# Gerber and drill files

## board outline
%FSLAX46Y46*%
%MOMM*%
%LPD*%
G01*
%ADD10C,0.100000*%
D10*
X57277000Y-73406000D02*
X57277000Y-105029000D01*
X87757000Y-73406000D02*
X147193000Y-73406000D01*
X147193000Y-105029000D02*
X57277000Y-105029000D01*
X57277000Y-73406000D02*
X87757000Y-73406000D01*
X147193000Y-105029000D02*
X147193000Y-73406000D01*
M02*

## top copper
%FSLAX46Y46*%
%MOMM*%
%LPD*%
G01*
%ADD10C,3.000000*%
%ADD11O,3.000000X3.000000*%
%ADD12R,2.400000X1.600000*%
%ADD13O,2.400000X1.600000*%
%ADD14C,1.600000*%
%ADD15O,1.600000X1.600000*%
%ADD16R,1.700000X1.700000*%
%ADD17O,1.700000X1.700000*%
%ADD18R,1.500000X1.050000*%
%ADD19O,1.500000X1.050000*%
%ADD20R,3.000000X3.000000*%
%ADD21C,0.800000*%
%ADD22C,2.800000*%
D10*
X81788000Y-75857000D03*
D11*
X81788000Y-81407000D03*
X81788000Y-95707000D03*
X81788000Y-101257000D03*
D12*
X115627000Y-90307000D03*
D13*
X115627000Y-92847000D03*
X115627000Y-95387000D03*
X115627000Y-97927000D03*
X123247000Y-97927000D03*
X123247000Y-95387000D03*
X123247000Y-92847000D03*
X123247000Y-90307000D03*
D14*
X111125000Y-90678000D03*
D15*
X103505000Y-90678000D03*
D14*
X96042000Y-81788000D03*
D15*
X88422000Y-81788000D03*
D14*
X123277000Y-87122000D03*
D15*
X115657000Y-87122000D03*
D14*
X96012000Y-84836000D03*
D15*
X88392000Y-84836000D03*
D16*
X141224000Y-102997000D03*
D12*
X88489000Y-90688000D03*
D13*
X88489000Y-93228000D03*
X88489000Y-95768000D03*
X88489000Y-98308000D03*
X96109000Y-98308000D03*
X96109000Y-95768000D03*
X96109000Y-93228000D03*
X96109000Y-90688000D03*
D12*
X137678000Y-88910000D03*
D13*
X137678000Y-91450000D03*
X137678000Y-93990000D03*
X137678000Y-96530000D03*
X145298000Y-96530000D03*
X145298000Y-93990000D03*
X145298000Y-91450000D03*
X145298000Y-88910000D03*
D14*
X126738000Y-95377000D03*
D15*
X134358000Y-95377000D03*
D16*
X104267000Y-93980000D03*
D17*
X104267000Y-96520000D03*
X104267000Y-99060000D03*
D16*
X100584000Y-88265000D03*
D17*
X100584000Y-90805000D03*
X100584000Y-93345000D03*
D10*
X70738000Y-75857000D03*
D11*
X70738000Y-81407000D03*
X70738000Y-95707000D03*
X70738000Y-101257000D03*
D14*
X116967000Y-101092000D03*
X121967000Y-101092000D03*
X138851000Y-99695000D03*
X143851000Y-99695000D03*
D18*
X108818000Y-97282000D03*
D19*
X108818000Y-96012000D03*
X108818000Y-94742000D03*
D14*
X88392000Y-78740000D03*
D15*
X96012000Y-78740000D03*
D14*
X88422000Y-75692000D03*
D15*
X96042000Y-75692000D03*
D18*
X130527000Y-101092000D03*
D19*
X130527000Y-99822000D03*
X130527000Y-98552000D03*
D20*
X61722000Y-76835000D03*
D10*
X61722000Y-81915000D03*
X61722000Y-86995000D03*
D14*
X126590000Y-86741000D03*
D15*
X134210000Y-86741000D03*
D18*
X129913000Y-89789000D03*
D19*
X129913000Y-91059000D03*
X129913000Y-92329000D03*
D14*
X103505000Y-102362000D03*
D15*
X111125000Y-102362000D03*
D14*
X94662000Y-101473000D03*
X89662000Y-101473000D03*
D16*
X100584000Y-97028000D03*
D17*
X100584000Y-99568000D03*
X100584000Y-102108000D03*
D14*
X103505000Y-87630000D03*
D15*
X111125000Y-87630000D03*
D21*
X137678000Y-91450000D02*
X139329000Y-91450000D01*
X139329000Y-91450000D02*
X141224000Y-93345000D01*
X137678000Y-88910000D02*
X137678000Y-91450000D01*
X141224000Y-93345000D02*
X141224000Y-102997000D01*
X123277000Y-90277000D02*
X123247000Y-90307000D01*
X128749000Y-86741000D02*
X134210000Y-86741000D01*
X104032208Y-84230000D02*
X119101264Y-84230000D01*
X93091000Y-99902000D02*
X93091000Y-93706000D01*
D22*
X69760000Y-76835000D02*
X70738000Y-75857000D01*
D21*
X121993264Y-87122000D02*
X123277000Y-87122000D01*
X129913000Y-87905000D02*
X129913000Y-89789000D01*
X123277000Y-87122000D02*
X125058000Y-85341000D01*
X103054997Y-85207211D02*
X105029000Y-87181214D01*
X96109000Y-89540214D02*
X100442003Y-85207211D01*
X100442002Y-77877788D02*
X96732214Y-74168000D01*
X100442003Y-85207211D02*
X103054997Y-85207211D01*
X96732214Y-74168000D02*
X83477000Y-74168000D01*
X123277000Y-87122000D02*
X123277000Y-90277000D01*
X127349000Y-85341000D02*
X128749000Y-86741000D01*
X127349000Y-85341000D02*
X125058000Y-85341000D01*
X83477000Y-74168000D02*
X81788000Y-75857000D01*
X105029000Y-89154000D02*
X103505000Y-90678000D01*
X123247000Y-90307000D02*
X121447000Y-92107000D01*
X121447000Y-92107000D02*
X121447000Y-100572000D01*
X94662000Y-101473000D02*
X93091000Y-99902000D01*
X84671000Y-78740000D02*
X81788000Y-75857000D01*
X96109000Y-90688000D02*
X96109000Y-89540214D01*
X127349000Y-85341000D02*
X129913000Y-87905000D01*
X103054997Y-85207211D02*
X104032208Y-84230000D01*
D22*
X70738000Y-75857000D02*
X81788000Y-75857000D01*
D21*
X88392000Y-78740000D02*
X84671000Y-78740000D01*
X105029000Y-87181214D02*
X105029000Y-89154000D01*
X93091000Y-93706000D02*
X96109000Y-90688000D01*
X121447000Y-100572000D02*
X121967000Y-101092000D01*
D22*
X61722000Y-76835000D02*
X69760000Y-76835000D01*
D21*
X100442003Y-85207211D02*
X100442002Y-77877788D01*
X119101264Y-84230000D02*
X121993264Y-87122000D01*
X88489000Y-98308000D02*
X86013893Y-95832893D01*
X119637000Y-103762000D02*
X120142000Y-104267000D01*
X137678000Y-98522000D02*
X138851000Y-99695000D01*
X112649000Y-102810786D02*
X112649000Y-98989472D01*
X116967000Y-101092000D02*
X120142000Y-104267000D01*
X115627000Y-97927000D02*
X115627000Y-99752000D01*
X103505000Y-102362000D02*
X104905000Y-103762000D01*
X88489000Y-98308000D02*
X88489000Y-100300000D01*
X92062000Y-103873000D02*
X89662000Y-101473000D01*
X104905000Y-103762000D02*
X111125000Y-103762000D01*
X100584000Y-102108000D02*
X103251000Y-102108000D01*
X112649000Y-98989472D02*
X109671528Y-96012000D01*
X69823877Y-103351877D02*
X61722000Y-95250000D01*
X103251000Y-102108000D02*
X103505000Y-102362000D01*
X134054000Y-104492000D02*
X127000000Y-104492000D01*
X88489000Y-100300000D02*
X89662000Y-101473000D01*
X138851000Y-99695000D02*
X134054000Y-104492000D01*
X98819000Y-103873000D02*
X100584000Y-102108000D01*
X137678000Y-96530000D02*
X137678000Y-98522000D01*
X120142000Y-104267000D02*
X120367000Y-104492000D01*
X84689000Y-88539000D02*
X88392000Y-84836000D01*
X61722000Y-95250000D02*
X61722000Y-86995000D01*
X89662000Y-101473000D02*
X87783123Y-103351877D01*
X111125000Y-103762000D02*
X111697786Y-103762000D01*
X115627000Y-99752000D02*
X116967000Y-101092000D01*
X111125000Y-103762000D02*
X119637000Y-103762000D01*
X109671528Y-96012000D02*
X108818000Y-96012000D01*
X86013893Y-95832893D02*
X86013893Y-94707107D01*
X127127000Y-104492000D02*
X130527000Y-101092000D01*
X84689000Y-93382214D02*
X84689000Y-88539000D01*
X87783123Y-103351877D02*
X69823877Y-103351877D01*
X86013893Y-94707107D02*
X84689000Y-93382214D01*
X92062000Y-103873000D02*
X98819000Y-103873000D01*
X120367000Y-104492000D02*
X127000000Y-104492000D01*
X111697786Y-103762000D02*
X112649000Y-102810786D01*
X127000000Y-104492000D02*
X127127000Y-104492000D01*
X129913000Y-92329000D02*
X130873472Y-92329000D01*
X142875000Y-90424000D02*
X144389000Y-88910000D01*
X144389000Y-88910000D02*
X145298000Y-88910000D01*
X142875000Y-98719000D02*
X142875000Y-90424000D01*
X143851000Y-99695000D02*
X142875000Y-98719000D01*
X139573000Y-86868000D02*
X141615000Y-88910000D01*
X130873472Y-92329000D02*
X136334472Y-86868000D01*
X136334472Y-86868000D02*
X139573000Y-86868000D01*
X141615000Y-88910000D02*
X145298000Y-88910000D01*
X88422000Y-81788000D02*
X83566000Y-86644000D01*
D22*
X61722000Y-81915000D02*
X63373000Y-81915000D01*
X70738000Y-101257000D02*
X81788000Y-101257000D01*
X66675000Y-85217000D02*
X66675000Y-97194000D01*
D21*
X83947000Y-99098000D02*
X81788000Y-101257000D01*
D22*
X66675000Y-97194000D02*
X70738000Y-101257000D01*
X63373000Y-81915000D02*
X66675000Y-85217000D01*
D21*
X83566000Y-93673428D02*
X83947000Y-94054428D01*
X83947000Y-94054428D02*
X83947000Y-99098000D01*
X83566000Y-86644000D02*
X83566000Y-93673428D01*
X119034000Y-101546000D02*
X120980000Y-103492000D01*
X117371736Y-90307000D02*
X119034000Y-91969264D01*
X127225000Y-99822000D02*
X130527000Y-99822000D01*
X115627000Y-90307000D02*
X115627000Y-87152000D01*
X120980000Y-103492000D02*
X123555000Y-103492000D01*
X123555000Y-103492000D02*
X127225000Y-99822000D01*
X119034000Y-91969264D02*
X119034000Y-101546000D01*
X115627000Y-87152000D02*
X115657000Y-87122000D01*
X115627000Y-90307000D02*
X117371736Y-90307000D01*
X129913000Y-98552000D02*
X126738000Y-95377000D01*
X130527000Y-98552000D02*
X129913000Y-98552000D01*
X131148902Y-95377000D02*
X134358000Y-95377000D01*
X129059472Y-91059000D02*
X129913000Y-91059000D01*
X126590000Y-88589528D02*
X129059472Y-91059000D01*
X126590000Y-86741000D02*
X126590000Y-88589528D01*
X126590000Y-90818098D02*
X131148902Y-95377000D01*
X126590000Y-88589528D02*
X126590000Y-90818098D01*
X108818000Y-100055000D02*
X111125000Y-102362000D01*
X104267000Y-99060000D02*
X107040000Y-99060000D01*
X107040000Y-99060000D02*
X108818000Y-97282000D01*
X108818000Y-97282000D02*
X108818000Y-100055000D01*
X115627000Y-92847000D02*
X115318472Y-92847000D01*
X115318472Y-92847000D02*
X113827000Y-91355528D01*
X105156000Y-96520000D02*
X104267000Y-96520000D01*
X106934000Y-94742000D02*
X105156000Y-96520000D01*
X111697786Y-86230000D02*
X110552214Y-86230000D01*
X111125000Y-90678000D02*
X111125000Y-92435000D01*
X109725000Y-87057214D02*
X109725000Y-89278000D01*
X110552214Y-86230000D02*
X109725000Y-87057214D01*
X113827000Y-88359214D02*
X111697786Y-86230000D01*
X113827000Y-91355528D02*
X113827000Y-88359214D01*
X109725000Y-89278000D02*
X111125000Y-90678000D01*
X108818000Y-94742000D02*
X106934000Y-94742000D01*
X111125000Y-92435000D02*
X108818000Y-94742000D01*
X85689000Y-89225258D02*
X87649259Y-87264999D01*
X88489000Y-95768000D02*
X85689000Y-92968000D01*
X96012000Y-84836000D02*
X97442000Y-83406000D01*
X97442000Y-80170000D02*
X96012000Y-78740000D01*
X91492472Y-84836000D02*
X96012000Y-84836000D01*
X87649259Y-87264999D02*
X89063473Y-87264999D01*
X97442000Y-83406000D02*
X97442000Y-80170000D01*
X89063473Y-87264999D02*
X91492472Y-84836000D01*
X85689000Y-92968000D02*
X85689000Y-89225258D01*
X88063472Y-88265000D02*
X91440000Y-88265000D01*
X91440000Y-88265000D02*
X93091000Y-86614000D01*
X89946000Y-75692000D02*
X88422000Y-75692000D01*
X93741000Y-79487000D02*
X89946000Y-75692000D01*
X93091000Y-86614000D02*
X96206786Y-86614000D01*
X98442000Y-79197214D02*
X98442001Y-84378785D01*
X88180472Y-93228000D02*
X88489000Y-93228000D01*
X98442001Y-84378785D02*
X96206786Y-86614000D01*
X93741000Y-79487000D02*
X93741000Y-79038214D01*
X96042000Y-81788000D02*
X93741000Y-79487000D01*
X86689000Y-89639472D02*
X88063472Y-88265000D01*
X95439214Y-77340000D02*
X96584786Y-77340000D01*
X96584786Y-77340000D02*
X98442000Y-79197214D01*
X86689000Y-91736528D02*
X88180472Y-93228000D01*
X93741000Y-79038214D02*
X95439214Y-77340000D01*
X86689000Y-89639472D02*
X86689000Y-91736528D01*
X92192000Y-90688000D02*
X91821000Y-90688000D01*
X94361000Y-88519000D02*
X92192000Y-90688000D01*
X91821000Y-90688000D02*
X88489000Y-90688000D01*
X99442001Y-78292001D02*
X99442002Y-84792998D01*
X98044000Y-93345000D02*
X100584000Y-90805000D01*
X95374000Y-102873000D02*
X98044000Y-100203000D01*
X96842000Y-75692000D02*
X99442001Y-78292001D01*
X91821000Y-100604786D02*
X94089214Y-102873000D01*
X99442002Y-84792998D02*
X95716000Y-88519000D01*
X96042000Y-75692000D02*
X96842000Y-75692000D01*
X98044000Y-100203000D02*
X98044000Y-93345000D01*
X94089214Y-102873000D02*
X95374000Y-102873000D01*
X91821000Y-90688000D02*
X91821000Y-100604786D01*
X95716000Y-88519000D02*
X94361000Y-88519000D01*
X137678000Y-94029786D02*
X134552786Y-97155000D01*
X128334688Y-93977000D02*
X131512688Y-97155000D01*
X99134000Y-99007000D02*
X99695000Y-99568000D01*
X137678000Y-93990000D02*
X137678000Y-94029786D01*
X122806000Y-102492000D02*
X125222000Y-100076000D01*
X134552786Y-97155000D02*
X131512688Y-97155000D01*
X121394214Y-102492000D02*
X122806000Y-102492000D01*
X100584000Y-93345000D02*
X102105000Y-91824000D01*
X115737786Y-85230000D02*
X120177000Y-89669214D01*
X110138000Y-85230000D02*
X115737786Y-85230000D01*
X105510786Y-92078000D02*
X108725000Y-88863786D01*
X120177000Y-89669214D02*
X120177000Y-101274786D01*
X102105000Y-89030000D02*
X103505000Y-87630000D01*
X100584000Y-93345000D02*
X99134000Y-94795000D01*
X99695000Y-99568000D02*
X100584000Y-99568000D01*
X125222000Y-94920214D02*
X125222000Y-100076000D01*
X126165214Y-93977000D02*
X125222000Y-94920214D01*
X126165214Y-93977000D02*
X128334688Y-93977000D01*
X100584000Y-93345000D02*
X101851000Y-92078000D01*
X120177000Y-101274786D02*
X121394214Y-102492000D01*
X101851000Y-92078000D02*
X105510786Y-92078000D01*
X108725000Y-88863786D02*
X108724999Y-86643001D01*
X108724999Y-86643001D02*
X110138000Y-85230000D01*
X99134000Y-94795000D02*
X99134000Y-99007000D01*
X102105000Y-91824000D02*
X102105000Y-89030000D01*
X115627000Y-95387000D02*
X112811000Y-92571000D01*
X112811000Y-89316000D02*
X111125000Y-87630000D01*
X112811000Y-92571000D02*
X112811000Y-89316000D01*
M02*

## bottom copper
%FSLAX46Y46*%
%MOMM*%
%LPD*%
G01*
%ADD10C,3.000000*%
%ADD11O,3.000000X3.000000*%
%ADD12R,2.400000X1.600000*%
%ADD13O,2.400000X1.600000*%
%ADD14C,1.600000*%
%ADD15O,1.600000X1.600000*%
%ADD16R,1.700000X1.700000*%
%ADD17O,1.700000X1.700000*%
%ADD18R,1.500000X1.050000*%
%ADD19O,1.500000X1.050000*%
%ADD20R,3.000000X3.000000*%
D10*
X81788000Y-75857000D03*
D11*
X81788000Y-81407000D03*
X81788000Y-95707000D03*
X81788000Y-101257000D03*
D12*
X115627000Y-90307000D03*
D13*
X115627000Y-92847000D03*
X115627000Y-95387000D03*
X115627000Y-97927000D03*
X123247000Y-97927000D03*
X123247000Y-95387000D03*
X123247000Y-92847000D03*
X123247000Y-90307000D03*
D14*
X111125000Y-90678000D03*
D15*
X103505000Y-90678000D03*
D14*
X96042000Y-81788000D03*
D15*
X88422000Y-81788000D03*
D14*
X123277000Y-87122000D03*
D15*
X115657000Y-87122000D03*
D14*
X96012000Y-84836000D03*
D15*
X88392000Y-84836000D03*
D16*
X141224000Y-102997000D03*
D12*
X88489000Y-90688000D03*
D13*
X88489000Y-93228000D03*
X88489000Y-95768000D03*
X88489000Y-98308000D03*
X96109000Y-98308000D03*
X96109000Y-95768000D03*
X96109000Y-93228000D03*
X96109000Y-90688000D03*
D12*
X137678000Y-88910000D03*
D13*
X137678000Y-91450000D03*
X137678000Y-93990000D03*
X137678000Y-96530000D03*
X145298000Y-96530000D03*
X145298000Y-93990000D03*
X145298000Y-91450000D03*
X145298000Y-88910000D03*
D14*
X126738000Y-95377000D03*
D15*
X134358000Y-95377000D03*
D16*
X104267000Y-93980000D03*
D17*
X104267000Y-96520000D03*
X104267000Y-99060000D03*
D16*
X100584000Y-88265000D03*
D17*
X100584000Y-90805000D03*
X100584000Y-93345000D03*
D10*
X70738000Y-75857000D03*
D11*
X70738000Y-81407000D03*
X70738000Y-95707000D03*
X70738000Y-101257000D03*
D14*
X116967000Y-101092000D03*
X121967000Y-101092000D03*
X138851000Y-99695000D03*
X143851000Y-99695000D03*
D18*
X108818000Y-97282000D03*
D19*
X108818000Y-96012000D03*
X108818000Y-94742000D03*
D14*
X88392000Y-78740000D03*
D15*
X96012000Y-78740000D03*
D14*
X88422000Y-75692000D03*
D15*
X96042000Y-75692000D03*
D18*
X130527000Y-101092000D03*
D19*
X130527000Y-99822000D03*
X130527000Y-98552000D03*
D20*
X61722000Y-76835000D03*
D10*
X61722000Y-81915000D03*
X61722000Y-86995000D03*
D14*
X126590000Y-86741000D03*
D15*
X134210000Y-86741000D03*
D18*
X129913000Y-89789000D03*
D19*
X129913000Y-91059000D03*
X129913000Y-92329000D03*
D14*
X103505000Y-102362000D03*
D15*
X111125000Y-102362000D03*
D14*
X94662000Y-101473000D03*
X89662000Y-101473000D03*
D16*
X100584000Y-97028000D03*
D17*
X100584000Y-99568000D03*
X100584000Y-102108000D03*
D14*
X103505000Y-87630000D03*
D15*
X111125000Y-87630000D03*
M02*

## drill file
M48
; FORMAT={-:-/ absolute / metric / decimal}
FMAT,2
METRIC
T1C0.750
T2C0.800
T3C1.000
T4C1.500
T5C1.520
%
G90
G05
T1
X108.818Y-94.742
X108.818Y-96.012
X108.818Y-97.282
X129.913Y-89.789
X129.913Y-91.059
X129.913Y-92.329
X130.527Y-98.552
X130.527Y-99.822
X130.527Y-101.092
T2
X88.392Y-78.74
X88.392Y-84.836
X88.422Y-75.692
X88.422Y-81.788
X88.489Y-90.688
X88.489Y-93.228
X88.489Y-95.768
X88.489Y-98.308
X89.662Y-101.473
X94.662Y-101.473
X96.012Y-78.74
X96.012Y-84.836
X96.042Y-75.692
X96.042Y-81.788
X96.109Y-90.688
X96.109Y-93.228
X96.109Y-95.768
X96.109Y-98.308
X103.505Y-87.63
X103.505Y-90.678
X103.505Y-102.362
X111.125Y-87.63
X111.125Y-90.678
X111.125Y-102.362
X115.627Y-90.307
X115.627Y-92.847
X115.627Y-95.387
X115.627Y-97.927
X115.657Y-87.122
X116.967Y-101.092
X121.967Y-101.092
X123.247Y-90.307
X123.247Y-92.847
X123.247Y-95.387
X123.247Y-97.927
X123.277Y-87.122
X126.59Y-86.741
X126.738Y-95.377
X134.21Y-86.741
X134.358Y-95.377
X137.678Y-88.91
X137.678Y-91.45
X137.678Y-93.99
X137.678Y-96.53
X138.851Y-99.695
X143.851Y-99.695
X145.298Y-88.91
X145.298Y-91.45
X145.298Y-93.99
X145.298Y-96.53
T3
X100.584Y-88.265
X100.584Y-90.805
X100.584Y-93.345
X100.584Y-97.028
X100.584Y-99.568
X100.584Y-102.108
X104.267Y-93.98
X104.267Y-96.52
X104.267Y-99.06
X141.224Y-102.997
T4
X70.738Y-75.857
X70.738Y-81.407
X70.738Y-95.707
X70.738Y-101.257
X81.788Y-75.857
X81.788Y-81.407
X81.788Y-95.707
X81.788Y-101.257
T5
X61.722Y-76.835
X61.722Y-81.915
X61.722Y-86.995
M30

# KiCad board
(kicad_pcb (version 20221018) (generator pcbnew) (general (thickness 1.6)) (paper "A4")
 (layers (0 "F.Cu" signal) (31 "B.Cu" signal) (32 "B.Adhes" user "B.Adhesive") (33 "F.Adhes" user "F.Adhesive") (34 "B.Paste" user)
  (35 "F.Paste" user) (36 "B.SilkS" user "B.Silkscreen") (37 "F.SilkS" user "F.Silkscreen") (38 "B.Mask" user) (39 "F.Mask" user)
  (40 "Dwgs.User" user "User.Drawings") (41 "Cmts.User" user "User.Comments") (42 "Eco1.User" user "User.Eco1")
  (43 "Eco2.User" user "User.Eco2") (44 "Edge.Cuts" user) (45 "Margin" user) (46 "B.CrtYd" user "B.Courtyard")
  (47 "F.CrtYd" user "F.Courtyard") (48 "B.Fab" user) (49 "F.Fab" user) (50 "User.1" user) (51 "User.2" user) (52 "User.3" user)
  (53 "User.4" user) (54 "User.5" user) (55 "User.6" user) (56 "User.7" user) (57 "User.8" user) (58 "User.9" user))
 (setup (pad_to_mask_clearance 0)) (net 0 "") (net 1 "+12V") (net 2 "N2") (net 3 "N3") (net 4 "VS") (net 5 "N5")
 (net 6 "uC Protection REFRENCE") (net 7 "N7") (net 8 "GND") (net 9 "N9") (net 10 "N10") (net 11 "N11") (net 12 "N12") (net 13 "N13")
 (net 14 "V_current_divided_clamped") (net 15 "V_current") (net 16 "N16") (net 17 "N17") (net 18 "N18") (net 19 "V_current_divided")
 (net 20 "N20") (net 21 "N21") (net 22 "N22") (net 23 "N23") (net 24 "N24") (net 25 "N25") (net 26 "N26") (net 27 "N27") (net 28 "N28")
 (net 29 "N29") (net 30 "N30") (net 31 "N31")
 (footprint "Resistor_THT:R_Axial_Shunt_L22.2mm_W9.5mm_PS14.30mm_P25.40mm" (layer "F.Cu") (at 81.788 75.857 -90)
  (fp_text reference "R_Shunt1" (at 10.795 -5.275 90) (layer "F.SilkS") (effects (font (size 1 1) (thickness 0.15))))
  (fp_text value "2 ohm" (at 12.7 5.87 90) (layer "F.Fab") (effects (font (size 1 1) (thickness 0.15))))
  (pad "1" thru_hole circle (at 0 0 270) (size 3 3) (drill 1.5) (layers "*.Cu" "*.Mask") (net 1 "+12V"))
  (pad "2" thru_hole oval (at 5.55 0 270) (size 3 3) (drill 1.5) (layers "*.Cu" "*.Mask") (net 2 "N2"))
  (pad "3" thru_hole oval (at 19.85 0 270) (size 3 3) (drill 1.5) (layers "*.Cu" "*.Mask") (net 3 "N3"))
  (pad "4" thru_hole oval (at 25.4 0 270) (size 3 3) (drill 1.5) (layers "*.Cu" "*.Mask") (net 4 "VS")))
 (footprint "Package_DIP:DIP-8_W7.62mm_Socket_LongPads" (layer "F.Cu") (at 115.627 90.307)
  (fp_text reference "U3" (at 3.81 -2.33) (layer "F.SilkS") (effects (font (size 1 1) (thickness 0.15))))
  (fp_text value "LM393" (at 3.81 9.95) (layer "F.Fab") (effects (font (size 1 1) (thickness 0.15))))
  (pad "1" thru_hole rect (at 0 0) (size 2.4 1.6) (drill 0.8) (layers "*.Cu" "*.Mask") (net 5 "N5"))
  (pad "2" thru_hole oval (at 0 2.54) (size 2.4 1.6) (drill 0.8) (layers "*.Cu" "*.Mask") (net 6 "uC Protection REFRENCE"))
  (pad "3" thru_hole oval (at 0 5.08) (size 2.4 1.6) (drill 0.8) (layers "*.Cu" "*.Mask") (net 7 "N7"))
  (pad "4" thru_hole oval (at 0 7.62) (size 2.4 1.6) (drill 0.8) (layers "*.Cu" "*.Mask") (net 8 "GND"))
  (pad "5" thru_hole oval (at 7.62 7.62) (size 2.4 1.6) (drill 0.8) (layers "*.Cu" "*.Mask") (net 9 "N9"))
  (pad "6" thru_hole oval (at 7.62 5.08) (size 2.4 1.6) (drill 0.8) (layers "*.Cu" "*.Mask") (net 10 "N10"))
  (pad "7" thru_hole oval (at 7.62 2.54) (size 2.4 1.6) (drill 0.8) (layers "*.Cu" "*.Mask") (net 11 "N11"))
  (pad "8" thru_hole oval (at 7.62 0) (size 2.4 1.6) (drill 0.8) (layers "*.Cu" "*.Mask") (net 1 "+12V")))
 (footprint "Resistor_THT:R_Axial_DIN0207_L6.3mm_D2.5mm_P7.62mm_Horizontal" (layer "F.Cu") (at 111.125 90.678 180)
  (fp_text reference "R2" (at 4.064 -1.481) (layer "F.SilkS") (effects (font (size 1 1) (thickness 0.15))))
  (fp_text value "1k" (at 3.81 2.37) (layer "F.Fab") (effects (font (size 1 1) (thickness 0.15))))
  (pad "1" thru_hole circle (at 0 0 180) (size 1.6 1.6) (drill 0.8) (layers "*.Cu" "*.Mask") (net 6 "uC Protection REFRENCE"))
  (pad "2" thru_hole oval (at 7.62 0 180) (size 1.6 1.6) (drill 0.8) (layers "*.Cu" "*.Mask") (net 1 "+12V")))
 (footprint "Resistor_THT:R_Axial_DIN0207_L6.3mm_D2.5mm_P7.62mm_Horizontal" (layer "F.Cu") (at 96.042 81.788 180)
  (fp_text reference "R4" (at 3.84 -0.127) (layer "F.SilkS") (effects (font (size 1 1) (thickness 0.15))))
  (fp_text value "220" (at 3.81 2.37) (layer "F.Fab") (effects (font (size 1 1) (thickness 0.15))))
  (pad "1" thru_hole circle (at 0 0 180) (size 1.6 1.6) (drill 0.8) (layers "*.Cu" "*.Mask") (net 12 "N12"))
  (pad "2" thru_hole oval (at 7.62 0 180) (size 1.6 1.6) (drill 0.8) (layers "*.Cu" "*.Mask") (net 4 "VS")))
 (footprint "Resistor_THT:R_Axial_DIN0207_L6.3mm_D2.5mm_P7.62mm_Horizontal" (layer "F.Cu") (at 123.277 87.122 180)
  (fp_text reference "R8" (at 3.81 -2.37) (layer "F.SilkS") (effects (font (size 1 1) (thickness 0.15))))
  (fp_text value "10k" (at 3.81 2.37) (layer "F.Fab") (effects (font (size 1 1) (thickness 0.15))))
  (pad "1" thru_hole circle (at 0 0 180) (size 1.6 1.6) (drill 0.8) (layers "*.Cu" "*.Mask") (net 1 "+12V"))
  (pad "2" thru_hole oval (at 7.62 0 180) (size 1.6 1.6) (drill 0.8) (layers "*.Cu" "*.Mask") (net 5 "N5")))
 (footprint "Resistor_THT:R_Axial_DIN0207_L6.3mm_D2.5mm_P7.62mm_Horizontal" (layer "F.Cu") (at 96.012 84.836 180)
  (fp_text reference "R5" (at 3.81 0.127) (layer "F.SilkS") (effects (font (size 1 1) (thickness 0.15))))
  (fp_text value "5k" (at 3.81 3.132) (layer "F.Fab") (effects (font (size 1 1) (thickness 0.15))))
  (pad "1" thru_hole circle (at 0 0 180) (size 1.6 1.6) (drill 0.8) (layers "*.Cu" "*.Mask") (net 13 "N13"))
  (pad "2" thru_hole oval (at 7.62 0 180) (size 1.6 1.6) (drill 0.8) (layers "*.Cu" "*.Mask") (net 8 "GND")))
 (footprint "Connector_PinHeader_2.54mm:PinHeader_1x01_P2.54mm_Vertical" (layer "F.Cu") (at 141.224 102.997)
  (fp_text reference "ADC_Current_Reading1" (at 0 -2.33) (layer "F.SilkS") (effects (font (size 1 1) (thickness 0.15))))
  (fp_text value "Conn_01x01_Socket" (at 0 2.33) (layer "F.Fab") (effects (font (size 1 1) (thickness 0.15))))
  (pad "1" thru_hole rect (at 0 0) (size 1.7 1.7) (drill 1) (layers "*.Cu" "*.Mask") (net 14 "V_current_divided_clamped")))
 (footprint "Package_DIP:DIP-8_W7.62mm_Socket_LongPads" (layer "F.Cu") (at 88.489 90.688)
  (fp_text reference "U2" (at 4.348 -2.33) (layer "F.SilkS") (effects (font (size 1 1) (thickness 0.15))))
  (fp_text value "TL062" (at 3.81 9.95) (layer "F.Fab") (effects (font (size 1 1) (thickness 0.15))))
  (pad "1" thru_hole rect (at 0 0) (size 2.4 1.6) (drill 0.8) (layers "*.Cu" "*.Mask") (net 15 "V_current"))
  (pad "2" thru_hole oval (at 0 2.54) (size 2.4 1.6) (drill 0.8) (layers "*.Cu" "*.Mask") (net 12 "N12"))
  (pad "3" thru_hole oval (at 0 5.08) (size 2.4 1.6) (drill 0.8) (layers "*.Cu" "*.Mask") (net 13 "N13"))
  (pad "4" thru_hole oval (at 0 7.62) (size 2.4 1.6) (drill 0.8) (layers "*.Cu" "*.Mask") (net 8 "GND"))
  (pad "5" thru_hole oval (at 7.62 7.62) (size 2.4 1.6) (drill 0.8) (layers "*.Cu" "*.Mask") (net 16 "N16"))
  (pad "6" thru_hole oval (at 7.62 5.08) (size 2.4 1.6) (drill 0.8) (layers "*.Cu" "*.Mask") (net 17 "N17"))
  (pad "7" thru_hole oval (at 7.62 2.54) (size 2.4 1.6) (drill 0.8) (layers "*.Cu" "*.Mask") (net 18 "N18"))
  (pad "8" thru_hole oval (at 7.62 0) (size 2.4 1.6) (drill 0.8) (layers "*.Cu" "*.Mask") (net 1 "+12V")))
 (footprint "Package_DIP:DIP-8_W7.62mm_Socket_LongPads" (layer "F.Cu") (at 137.678 88.91)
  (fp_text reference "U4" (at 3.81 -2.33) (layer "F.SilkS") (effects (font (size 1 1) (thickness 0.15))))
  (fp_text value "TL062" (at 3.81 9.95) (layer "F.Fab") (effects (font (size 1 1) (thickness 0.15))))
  (pad "1" thru_hole rect (at 0 0) (size 2.4 1.6) (drill 0.8) (layers "*.Cu" "*.Mask") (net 14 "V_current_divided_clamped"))
  (pad "2" thru_hole oval (at 0 2.54) (size 2.4 1.6) (drill 0.8) (layers "*.Cu" "*.Mask") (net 14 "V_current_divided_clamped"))
  (pad "3" thru_hole oval (at 0 5.08) (size 2.4 1.6) (drill 0.8) (layers "*.Cu" "*.Mask") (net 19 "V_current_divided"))
  (pad "4" thru_hole oval (at 0 7.62) (size 2.4 1.6) (drill 0.8) (layers "*.Cu" "*.Mask") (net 8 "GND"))
  (pad "5" thru_hole oval (at 7.62 7.62) (size 2.4 1.6) (drill 0.8) (layers "*.Cu" "*.Mask") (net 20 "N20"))
  (pad "6" thru_hole oval (at 7.62 5.08) (size 2.4 1.6) (drill 0.8) (layers "*.Cu" "*.Mask") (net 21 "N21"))
  (pad "7" thru_hole oval (at 7.62 2.54) (size 2.4 1.6) (drill 0.8) (layers "*.Cu" "*.Mask") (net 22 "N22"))
  (pad "8" thru_hole oval (at 7.62 0) (size 2.4 1.6) (drill 0.8) (layers "*.Cu" "*.Mask") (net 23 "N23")))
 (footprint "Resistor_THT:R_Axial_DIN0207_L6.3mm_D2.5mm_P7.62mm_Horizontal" (layer "F.Cu") (at 126.738 95.377)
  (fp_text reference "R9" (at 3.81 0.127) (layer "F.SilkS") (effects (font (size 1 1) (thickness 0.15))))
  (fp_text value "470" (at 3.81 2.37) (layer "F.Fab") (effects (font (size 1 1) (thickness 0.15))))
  (pad "1" thru_hole circle (at 0 0) (size 1.6 1.6) (drill 0.8) (layers "*.Cu" "*.Mask") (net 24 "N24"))
  (pad "2" thru_hole oval (at 7.62 0) (size 1.6 1.6) (drill 0.8) (layers "*.Cu" "*.Mask") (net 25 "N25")))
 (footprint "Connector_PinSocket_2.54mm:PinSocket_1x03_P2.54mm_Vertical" (layer "F.Cu") (at 104.267 93.98)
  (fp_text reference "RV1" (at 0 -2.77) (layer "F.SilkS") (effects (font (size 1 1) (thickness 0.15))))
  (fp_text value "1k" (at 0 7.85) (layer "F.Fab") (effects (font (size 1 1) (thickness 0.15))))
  (pad "1" thru_hole rect (at 0 0) (size 1.7 1.7) (drill 1) (layers "*.Cu" "*.Mask") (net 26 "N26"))
  (pad "2" thru_hole oval (at 0 2.54) (size 1.7 1.7) (drill 1) (layers "*.Cu" "*.Mask") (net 6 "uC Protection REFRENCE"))
  (pad "3" thru_hole oval (at 0 5.08) (size 1.7 1.7) (drill 1) (layers "*.Cu" "*.Mask") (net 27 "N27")))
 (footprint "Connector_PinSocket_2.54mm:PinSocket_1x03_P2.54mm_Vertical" (layer "F.Cu") (at 100.584 88.265)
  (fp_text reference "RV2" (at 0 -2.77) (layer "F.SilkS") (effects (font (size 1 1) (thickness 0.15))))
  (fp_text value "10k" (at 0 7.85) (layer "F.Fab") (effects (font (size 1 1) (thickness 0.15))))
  (pad "1" thru_hole rect (at 0 0) (size 1.7 1.7) (drill 1) (layers "*.Cu" "*.Mask") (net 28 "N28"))
  (pad "2" thru_hole oval (at 0 2.54) (size 1.7 1.7) (drill 1) (layers "*.Cu" "*.Mask") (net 15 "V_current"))
  (pad "3" thru_hole oval (at 0 5.08) (size 1.7 1.7) (drill 1) (layers "*.Cu" "*.Mask") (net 19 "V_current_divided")))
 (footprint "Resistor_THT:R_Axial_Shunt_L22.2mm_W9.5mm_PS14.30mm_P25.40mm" (layer "F.Cu") (at 70.738 75.857 -90)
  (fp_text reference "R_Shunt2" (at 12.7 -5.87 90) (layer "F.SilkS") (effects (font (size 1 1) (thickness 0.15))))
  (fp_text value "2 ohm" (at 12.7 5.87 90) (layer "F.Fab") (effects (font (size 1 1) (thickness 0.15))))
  (pad "1" thru_hole circle (at 0 0 270) (size 3 3) (drill 1.5) (layers "*.Cu" "*.Mask") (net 1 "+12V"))
  (pad "2" thru_hole oval (at 5.55 0 270) (size 3 3) (drill 1.5) (layers "*.Cu" "*.Mask") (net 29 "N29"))
  (pad "3" thru_hole oval (at 19.85 0 270) (size 3 3) (drill 1.5) (layers "*.Cu" "*.Mask") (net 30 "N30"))
  (pad "4" thru_hole oval (at 25.4 0 270) (size 3 3) (drill 1.5) (layers "*.Cu" "*.Mask") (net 4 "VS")))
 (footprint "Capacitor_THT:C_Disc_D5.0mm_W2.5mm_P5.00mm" (layer "F.Cu") (at 116.967 101.092)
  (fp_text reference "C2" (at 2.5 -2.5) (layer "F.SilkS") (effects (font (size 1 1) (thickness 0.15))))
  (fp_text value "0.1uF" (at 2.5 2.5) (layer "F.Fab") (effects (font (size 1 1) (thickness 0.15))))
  (pad "1" thru_hole circle (at 0 0) (size 1.6 1.6) (drill 0.8) (layers "*.Cu" "*.Mask") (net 8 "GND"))
  (pad "2" thru_hole circle (at 5 0) (size 1.6 1.6) (drill 0.8) (layers "*.Cu" "*.Mask") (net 1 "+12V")))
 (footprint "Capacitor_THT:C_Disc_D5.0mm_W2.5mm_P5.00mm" (layer "F.Cu") (at 138.851 99.695)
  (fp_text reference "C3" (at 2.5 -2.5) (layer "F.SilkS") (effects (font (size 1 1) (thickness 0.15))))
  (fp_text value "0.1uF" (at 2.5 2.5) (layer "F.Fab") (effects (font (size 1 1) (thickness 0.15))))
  (pad "1" thru_hole circle (at 0 0) (size 1.6 1.6) (drill 0.8) (layers "*.Cu" "*.Mask") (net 8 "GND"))
  (pad "2" thru_hole circle (at 5 0) (size 1.6 1.6) (drill 0.8) (layers "*.Cu" "*.Mask") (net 23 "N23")))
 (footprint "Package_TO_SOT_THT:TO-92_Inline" (layer "F.Cu") (at 108.818 97.282 90)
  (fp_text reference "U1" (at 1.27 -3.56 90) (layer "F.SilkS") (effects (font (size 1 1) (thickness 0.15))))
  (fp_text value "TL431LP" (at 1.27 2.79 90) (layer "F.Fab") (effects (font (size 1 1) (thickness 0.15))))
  (pad "1" thru_hole rect (at 0 0 90) (size 1.05 1.5) (drill 0.75) (layers "*.Cu" "*.Mask") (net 27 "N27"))
  (pad "2" thru_hole oval (at 1.27 0 90) (size 1.05 1.5) (drill 0.75) (layers "*.Cu" "*.Mask") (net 8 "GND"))
  (pad "3" thru_hole oval (at 2.54 0 90) (size 1.05 1.5) (drill 0.75) (layers "*.Cu" "*.Mask") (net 6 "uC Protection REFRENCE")))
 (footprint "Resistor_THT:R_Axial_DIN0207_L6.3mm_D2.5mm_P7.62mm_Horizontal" (layer "F.Cu") (at 88.392 78.74)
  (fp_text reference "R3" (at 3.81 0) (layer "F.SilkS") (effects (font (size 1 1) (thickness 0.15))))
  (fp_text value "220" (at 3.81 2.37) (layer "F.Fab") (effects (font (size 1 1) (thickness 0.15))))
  (pad "1" thru_hole circle (at 0 0) (size 1.6 1.6) (drill 0.8) (layers "*.Cu" "*.Mask") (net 1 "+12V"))
  (pad "2" thru_hole oval (at 7.62 0) (size 1.6 1.6) (drill 0.8) (layers "*.Cu" "*.Mask") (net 13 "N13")))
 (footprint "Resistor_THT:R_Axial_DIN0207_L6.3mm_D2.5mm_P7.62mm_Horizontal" (layer "F.Cu") (at 88.422 75.692)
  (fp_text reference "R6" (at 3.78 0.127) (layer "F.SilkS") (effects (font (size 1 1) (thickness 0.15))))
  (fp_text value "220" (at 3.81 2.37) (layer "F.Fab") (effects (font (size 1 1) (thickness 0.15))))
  (pad "1" thru_hole circle (at 0 0) (size 1.6 1.6) (drill 0.8) (layers "*.Cu" "*.Mask") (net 12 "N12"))
  (pad "2" thru_hole oval (at 7.62 0) (size 1.6 1.6) (drill 0.8) (layers "*.Cu" "*.Mask") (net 15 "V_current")))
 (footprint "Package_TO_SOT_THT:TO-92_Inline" (layer "F.Cu") (at 130.527 101.092 90)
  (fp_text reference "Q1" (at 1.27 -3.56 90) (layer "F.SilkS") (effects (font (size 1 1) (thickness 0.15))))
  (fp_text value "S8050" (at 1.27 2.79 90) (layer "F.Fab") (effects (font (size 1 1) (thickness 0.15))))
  (pad "1" thru_hole rect (at 0 0 90) (size 1.05 1.5) (drill 0.75) (layers "*.Cu" "*.Mask") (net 8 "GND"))
  (pad "2" thru_hole oval (at 1.27 0 90) (size 1.05 1.5) (drill 0.75) (layers "*.Cu" "*.Mask") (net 5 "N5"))
  (pad "3" thru_hole oval (at 2.54 0 90) (size 1.05 1.5) (drill 0.75) (layers "*.Cu" "*.Mask") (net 24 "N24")))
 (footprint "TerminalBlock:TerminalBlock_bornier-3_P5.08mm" (layer "F.Cu") (at 61.722 76.835 -90)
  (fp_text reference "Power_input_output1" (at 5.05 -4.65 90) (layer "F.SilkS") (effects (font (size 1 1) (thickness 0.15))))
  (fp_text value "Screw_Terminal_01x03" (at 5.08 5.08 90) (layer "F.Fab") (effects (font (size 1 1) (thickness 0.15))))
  (pad "1" thru_hole rect (at 0 0 270) (size 3 3) (drill 1.52) (layers "*.Cu" "*.Mask") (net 1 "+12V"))
  (pad "2" thru_hole circle (at 5.08 0 270) (size 3 3) (drill 1.52) (layers "*.Cu" "*.Mask") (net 4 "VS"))
  (pad "3" thru_hole circle (at 10.16 0 270) (size 3 3) (drill 1.52) (layers "*.Cu" "*.Mask") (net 8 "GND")))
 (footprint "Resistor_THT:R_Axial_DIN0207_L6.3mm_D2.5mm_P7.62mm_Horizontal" (layer "F.Cu") (at 126.59 86.741)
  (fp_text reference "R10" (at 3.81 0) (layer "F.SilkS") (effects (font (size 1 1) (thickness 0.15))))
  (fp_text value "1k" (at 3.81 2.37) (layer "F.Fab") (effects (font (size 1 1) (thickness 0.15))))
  (pad "1" thru_hole circle (at 0 0) (size 1.6 1.6) (drill 0.8) (layers "*.Cu" "*.Mask") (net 25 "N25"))
  (pad "2" thru_hole oval (at 7.62 0) (size 1.6 1.6) (drill 0.8) (layers "*.Cu" "*.Mask") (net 1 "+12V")))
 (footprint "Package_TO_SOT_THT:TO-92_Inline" (layer "F.Cu") (at 129.913 89.789 -90)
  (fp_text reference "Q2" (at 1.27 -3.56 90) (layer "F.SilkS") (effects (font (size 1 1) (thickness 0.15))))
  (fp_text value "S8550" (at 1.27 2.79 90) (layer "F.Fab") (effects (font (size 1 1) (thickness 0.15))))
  (pad "1" thru_hole rect (at 0 0 270) (size 1.05 1.5) (drill 0.75) (layers "*.Cu" "*.Mask") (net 1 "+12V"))
  (pad "2" thru_hole oval (at 1.27 0 270) (size 1.05 1.5) (drill 0.75) (layers "*.Cu" "*.Mask") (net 25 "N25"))
  (pad "3" thru_hole oval (at 2.54 0 270) (size 1.05 1.5) (drill 0.75) (layers "*.Cu" "*.Mask") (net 23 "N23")))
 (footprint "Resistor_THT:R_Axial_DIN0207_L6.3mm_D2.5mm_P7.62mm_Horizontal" (layer "F.Cu") (at 103.505 102.362)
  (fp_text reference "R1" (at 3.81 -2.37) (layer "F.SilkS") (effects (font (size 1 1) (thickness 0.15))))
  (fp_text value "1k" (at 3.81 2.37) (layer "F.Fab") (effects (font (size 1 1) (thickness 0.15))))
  (pad "1" thru_hole circle (at 0 0) (size 1.6 1.6) (drill 0.8) (layers "*.Cu" "*.Mask") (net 8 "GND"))
  (pad "2" thru_hole oval (at 7.62 0) (size 1.6 1.6) (drill 0.8) (layers "*.Cu" "*.Mask") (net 27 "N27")))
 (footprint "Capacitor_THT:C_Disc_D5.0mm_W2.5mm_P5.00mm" (layer "F.Cu") (at 94.662 101.473 180)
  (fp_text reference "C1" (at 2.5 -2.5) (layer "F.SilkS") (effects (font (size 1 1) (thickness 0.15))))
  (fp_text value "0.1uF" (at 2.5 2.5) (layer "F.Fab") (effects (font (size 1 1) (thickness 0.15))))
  (pad "1" thru_hole circle (at 0 0 180) (size 1.6 1.6) (drill 0.8) (layers "*.Cu" "*.Mask") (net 1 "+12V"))
  (pad "2" thru_hole circle (at 5 0 180) (size 1.6 1.6) (drill 0.8) (layers "*.Cu" "*.Mask") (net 8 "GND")))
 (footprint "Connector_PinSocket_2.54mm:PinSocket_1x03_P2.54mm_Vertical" (layer "F.Cu") (at 100.584 97.028)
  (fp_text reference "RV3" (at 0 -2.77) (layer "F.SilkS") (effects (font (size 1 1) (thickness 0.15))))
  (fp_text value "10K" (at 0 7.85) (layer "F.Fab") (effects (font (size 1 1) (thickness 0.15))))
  (pad "1" thru_hole rect (at 0 0) (size 1.7 1.7) (drill 1) (layers "*.Cu" "*.Mask") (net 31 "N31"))
  (pad "2" thru_hole oval (at 0 2.54) (size 1.7 1.7) (drill 1) (layers "*.Cu" "*.Mask") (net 19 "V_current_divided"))
  (pad "3" thru_hole oval (at 0 5.08) (size 1.7 1.7) (drill 1) (layers "*.Cu" "*.Mask") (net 8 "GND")))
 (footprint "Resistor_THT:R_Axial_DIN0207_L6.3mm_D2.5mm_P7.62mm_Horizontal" (layer "F.Cu") (at 103.505 87.63)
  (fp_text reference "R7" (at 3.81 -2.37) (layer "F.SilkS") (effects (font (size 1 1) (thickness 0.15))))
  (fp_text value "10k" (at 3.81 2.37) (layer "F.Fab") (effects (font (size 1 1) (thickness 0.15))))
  (pad "1" thru_hole circle (at 0 0) (size 1.6 1.6) (drill 0.8) (layers "*.Cu" "*.Mask") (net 19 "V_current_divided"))
  (pad "2" thru_hole oval (at 7.62 0) (size 1.6 1.6) (drill 0.8) (layers "*.Cu" "*.Mask") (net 7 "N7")))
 (gr_line (start 57.277 73.406) (end 57.277 105.029) (stroke (width 0.1) (type default)) (layer "Edge.Cuts"))
 (gr_line (start 87.757 73.406) (end 147.193 73.406) (stroke (width 0.1) (type default)) (layer "Edge.Cuts"))
 (gr_line (start 147.193 105.029) (end 57.277 105.029) (stroke (width 0.1) (type default)) (layer "Edge.Cuts"))
 (gr_line (start 57.277 73.406) (end 87.757 73.406) (stroke (width 0.1) (type default)) (layer "Edge.Cuts"))
 (gr_line (start 147.193 105.029) (end 147.193 73.406) (stroke (width 0.1) (type default)) (layer "Edge.Cuts"))
 (segment (start 137.678 91.45) (end 139.329 91.45) (width 0.8) (layer "F.Cu") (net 14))
 (segment (start 139.329 91.45) (end 141.224 93.345) (width 0.8) (layer "F.Cu") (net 14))
 (segment (start 137.678 88.91) (end 137.678 91.45) (width 0.8) (layer "F.Cu") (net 14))
 (segment (start 141.224 93.345) (end 141.224 102.997) (width 0.8) (layer "F.Cu") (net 14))
 (segment (start 123.277 90.277) (end 123.247 90.307) (width 0.8) (layer "F.Cu") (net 1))
 (segment (start 128.749 86.741) (end 134.21 86.741) (width 0.8) (layer "F.Cu") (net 1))
 (segment (start 104.032208 84.23) (end 119.101264 84.23) (width 0.8) (layer "F.Cu") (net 1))
 (segment (start 93.091 99.902) (end 93.091 93.706) (width 0.8) (layer "F.Cu") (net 1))
 (segment (start 69.76 76.835) (end 70.738 75.857) (width 2.8) (layer "F.Cu") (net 1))
 (segment (start 121.993264 87.122) (end 123.277 87.122) (width 0.8) (layer "F.Cu") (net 1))
 (segment (start 129.913 87.905) (end 129.913 89.789) (width 0.8) (layer "F.Cu") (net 1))
 (segment (start 123.277 87.122) (end 125.058 85.341) (width 0.8) (layer "F.Cu") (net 1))
 (segment (start 103.054997 85.207211) (end 105.029 87.181214) (width 0.8) (layer "F.Cu") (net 1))
 (segment (start 96.109 89.540214) (end 100.442003 85.207211) (width 0.8) (layer "F.Cu") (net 1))
 (segment (start 100.442002 77.877788) (end 96.732214 74.168) (width 0.8) (layer "F.Cu") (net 1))
 (segment (start 100.442003 85.207211) (end 103.054997 85.207211) (width 0.8) (layer "F.Cu") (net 1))
 (segment (start 96.732214 74.168) (end 83.477 74.168) (width 0.8) (layer "F.Cu") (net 1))
 (segment (start 123.277 87.122) (end 123.277 90.277) (width 0.8) (layer "F.Cu") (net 1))
 (segment (start 127.349 85.341) (end 128.749 86.741) (width 0.8) (layer "F.Cu") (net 1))
 (segment (start 127.349 85.341) (end 125.058 85.341) (width 0.8) (layer "F.Cu") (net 1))
 (segment (start 83.477 74.168) (end 81.788 75.857) (width 0.8) (layer "F.Cu") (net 1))
 (segment (start 105.029 89.154) (end 103.505 90.678) (width 0.8) (layer "F.Cu") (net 1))
 (segment (start 123.247 90.307) (end 121.447 92.107) (width 0.8) (layer "F.Cu") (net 1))
 (segment (start 121.447 92.107) (end 121.447 100.572) (width 0.8) (layer "F.Cu") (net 1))
 (segment (start 94.662 101.473) (end 93.091 99.902) (width 0.8) (layer "F.Cu") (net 1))
 (segment (start 84.671 78.74) (end 81.788 75.857) (width 0.8) (layer "F.Cu") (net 1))
 (segment (start 96.109 90.688) (end 96.109 89.540214) (width 0.8) (layer "F.Cu") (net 1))
 (segment (start 127.349 85.341) (end 129.913 87.905) (width 0.8) (layer "F.Cu") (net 1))
 (segment (start 103.054997 85.207211) (end 104.032208 84.23) (width 0.8) (layer "F.Cu") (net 1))
 (segment (start 70.738 75.857) (end 81.788 75.857) (width 2.8) (layer "F.Cu") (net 1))
 (segment (start 88.392 78.74) (end 84.671 78.74) (width 0.8) (layer "F.Cu") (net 1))
 (segment (start 105.029 87.181214) (end 105.029 89.154) (width 0.8) (layer "F.Cu") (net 1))
 (segment (start 93.091 93.706) (end 96.109 90.688) (width 0.8) (layer "F.Cu") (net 1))
 (segment (start 121.447 100.572) (end 121.967 101.092) (width 0.8) (layer "F.Cu") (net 1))
 (segment (start 61.722 76.835) (end 69.76 76.835) (width 2.8) (layer "F.Cu") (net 1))
 (segment (start 100.442003 85.207211) (end 100.442002 77.877788) (width 0.8) (layer "F.Cu") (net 1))
 (segment (start 119.101264 84.23) (end 121.993264 87.122) (width 0.8) (layer "F.Cu") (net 1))
 (segment (start 88.489 98.308) (end 86.013893 95.832893) (width 0.8) (layer "F.Cu") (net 8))
 (segment (start 119.637 103.762) (end 120.142 104.267) (width 0.8) (layer "F.Cu") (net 8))
 (segment (start 137.678 98.522) (end 138.851 99.695) (width 0.8) (layer "F.Cu") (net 8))
 (segment (start 112.649 102.810786) (end 112.649 98.989472) (width 0.8) (layer "F.Cu") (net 8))
 (segment (start 116.967 101.092) (end 120.142 104.267) (width 0.8) (layer "F.Cu") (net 8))
 (segment (start 115.627 97.927) (end 115.627 99.752) (width 0.8) (layer "F.Cu") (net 8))
 (segment (start 103.505 102.362) (end 104.905 103.762) (width 0.8) (layer "F.Cu") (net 8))
 (segment (start 88.489 98.308) (end 88.489 100.3) (width 0.8) (layer "F.Cu") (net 8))
 (segment (start 92.062 103.873) (end 89.662 101.473) (width 0.8) (layer "F.Cu") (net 8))
 (segment (start 104.905 103.762) (end 111.125 103.762) (width 0.8) (layer "F.Cu") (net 8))
 (segment (start 100.584 102.108) (end 103.251 102.108) (width 0.8) (layer "F.Cu") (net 8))
 (segment (start 112.649 98.989472) (end 109.671528 96.012) (width 0.8) (layer "F.Cu") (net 8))
 (segment (start 69.823877 103.351877) (end 61.722 95.25) (width 0.8) (layer "F.Cu") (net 8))
 (segment (start 103.251 102.108) (end 103.505 102.362) (width 0.8) (layer "F.Cu") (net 8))
 (segment (start 134.054 104.492) (end 127 104.492) (width 0.8) (layer "F.Cu") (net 8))
 (segment (start 88.489 100.3) (end 89.662 101.473) (width 0.8) (layer "F.Cu") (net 8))
 (segment (start 138.851 99.695) (end 134.054 104.492) (width 0.8) (layer "F.Cu") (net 8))
 (segment (start 98.819 103.873) (end 100.584 102.108) (width 0.8) (layer "F.Cu") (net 8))
 (segment (start 137.678 96.53) (end 137.678 98.522) (width 0.8) (layer "F.Cu") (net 8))
 (segment (start 120.142 104.267) (end 120.367 104.492) (width 0.8) (layer "F.Cu") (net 8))
 (segment (start 84.689 88.539) (end 88.392 84.836) (width 0.8) (layer "F.Cu") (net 8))
 (segment (start 61.722 95.25) (end 61.722 86.995) (width 0.8) (layer "F.Cu") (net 8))
 (segment (start 89.662 101.473) (end 87.783123 103.351877) (width 0.8) (layer "F.Cu") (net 8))
 (segment (start 111.125 103.762) (end 111.697786 103.762) (width 0.8) (layer "F.Cu") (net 8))
 (segment (start 115.627 99.752) (end 116.967 101.092) (width 0.8) (layer "F.Cu") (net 8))
 (segment (start 111.125 103.762) (end 119.637 103.762) (width 0.8) (layer "F.Cu") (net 8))
 (segment (start 109.671528 96.012) (end 108.818 96.012) (width 0.8) (layer "F.Cu") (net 8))
 (segment (start 86.013893 95.832893) (end 86.013893 94.707107) (width 0.8) (layer "F.Cu") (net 8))
 (segment (start 127.127 104.492) (end 130.527 101.092) (width 0.8) (layer "F.Cu") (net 8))
 (segment (start 84.689 93.382214) (end 84.689 88.539) (width 0.8) (layer "F.Cu") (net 8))
 (segment (start 87.783123 103.351877) (end 69.823877 103.351877) (width 0.8) (layer "F.Cu") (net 8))
 (segment (start 86.013893 94.707107) (end 84.689 93.382214) (width 0.8) (layer "F.Cu") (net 8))
 (segment (start 92.062 103.873) (end 98.819 103.873) (width 0.8) (layer "F.Cu") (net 8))
 (segment (start 120.367 104.492) (end 127 104.492) (width 0.8) (layer "F.Cu") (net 8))
 (segment (start 111.697786 103.762) (end 112.649 102.810786) (width 0.8) (layer "F.Cu") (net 8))
 (segment (start 127 104.492) (end 127.127 104.492) (width 0.8) (layer "F.Cu") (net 8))
 (segment (start 129.913 92.329) (end 130.873472 92.329) (width 0.8) (layer "F.Cu") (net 23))
 (segment (start 142.875 90.424) (end 144.389 88.91) (width 0.8) (layer "F.Cu") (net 23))
 (segment (start 144.389 88.91) (end 145.298 88.91) (width 0.8) (layer "F.Cu") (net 23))
 (segment (start 142.875 98.719) (end 142.875 90.424) (width 0.8) (layer "F.Cu") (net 23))
 (segment (start 143.851 99.695) (end 142.875 98.719) (width 0.8) (layer "F.Cu") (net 23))
 (segment (start 139.573 86.868) (end 141.615 88.91) (width 0.8) (layer "F.Cu") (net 23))
 (segment (start 130.873472 92.329) (end 136.334472 86.868) (width 0.8) (layer "F.Cu") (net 23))
 (segment (start 136.334472 86.868) (end 139.573 86.868) (width 0.8) (layer "F.Cu") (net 23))
 (segment (start 141.615 88.91) (end 145.298 88.91) (width 0.8) (layer "F.Cu") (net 23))
 (segment (start 88.422 81.788) (end 83.566 86.644) (width 0.8) (layer "F.Cu") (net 4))
 (segment (start 61.722 81.915) (end 63.373 81.915) (width 2.8) (layer "F.Cu") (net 4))
 (segment (start 70.738 101.257) (end 81.788 101.257) (width 2.8) (layer "F.Cu") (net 4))
 (segment (start 66.675 85.217) (end 66.675 97.194) (width 2.8) (layer "F.Cu") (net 4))
 (segment (start 83.947 99.098) (end 81.788 101.257) (width 0.8) (layer "F.Cu") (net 4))
 (segment (start 66.675 97.194) (end 70.738 101.257) (width 2.8) (layer "F.Cu") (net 4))
 (segment (start 63.373 81.915) (end 66.675 85.217) (width 2.8) (layer "F.Cu") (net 4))
 (segment (start 83.566 93.673428) (end 83.947 94.054428) (width 0.8) (layer "F.Cu") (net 4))
 (segment (start 83.947 94.054428) (end 83.947 99.098) (width 0.8) (layer "F.Cu") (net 4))
 (segment (start 83.566 86.644) (end 83.566 93.673428) (width 0.8) (layer "F.Cu") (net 4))
 (segment (start 119.034 101.546) (end 120.98 103.492) (width 0.8) (layer "F.Cu") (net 5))
 (segment (start 117.371736 90.307) (end 119.034 91.969264) (width 0.8) (layer "F.Cu") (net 5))
 (segment (start 127.225 99.822) (end 130.527 99.822) (width 0.8) (layer "F.Cu") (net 5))
 (segment (start 115.627 90.307) (end 115.627 87.152) (width 0.8) (layer "F.Cu") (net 5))
 (segment (start 120.98 103.492) (end 123.555 103.492) (width 0.8) (layer "F.Cu") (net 5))
 (segment (start 123.555 103.492) (end 127.225 99.822) (width 0.8) (layer "F.Cu") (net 5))
 (segment (start 119.034 91.969264) (end 119.034 101.546) (width 0.8) (layer "F.Cu") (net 5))
 (segment (start 115.627 87.152) (end 115.657 87.122) (width 0.8) (layer "F.Cu") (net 5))
 (segment (start 115.627 90.307) (end 117.371736 90.307) (width 0.8) (layer "F.Cu") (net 5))
 (segment (start 129.913 98.552) (end 126.738 95.377) (width 0.8) (layer "F.Cu") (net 24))
 (segment (start 130.527 98.552) (end 129.913 98.552) (width 0.8) (layer "F.Cu") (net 24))
 (segment (start 131.148902 95.377) (end 134.358 95.377) (width 0.8) (layer "F.Cu") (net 25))
 (segment (start 129.059472 91.059) (end 129.913 91.059) (width 0.8) (layer "F.Cu") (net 25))
 (segment (start 126.59 88.589528) (end 129.059472 91.059) (width 0.8) (layer "F.Cu") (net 25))
 (segment (start 126.59 86.741) (end 126.59 88.589528) (width 0.8) (layer "F.Cu") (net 25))
 (segment (start 126.59 90.818098) (end 131.148902 95.377) (width 0.8) (layer "F.Cu") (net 25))
 (segment (start 126.59 88.589528) (end 126.59 90.818098) (width 0.8) (layer "F.Cu") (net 25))
 (segment (start 108.818 100.055) (end 111.125 102.362) (width 0.8) (layer "F.Cu") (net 27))
 (segment (start 104.267 99.06) (end 107.04 99.06) (width 0.8) (layer "F.Cu") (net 27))
 (segment (start 107.04 99.06) (end 108.818 97.282) (width 0.8) (layer "F.Cu") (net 27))
 (segment (start 108.818 97.282) (end 108.818 100.055) (width 0.8) (layer "F.Cu") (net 27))
 (segment (start 115.627 92.847) (end 115.318472 92.847) (width 0.8) (layer "F.Cu") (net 6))
 (segment (start 115.318472 92.847) (end 113.827 91.355528) (width 0.8) (layer "F.Cu") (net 6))
 (segment (start 105.156 96.52) (end 104.267 96.52) (width 0.8) (layer "F.Cu") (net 6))
 (segment (start 106.934 94.742) (end 105.156 96.52) (width 0.8) (layer "F.Cu") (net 6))
 (segment (start 111.697786 86.23) (end 110.552214 86.23) (width 0.8) (layer "F.Cu") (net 6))
 (segment (start 111.125 90.678) (end 111.125 92.435) (width 0.8) (layer "F.Cu") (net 6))
 (segment (start 109.725 87.057214) (end 109.725 89.278) (width 0.8) (layer "F.Cu") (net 6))
 (segment (start 110.552214 86.23) (end 109.725 87.057214) (width 0.8) (layer "F.Cu") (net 6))
 (segment (start 113.827 88.359214) (end 111.697786 86.23) (width 0.8) (layer "F.Cu") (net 6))
 (segment (start 113.827 91.355528) (end 113.827 88.359214) (width 0.8) (layer "F.Cu") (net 6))
 (segment (start 109.725 89.278) (end 111.125 90.678) (width 0.8) (layer "F.Cu") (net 6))
 (segment (start 108.818 94.742) (end 106.934 94.742) (width 0.8) (layer "F.Cu") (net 6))
 (segment (start 111.125 92.435) (end 108.818 94.742) (width 0.8) (layer "F.Cu") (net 6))
 (segment (start 85.689 89.225258) (end 87.649259 87.264999) (width 0.8) (layer "F.Cu") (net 13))
 (segment (start 88.489 95.768) (end 85.689 92.968) (width 0.8) (layer "F.Cu") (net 13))
 (segment (start 96.012 84.836) (end 97.442 83.406) (width 0.8) (layer "F.Cu") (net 13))
 (segment (start 97.442 80.17) (end 96.012 78.74) (width 0.8) (layer "F.Cu") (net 13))
 (segment (start 91.492472 84.836) (end 96.012 84.836) (width 0.8) (layer "F.Cu") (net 13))
 (segment (start 87.649259 87.264999) (end 89.063473 87.264999) (width 0.8) (layer "F.Cu") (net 13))
 (segment (start 97.442 83.406) (end 97.442 80.17) (width 0.8) (layer "F.Cu") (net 13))
 (segment (start 89.063473 87.264999) (end 91.492472 84.836) (width 0.8) (layer "F.Cu") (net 13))
 (segment (start 85.689 92.968) (end 85.689 89.225258) (width 0.8) (layer "F.Cu") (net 13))
 (segment (start 88.063472 88.265) (end 91.44 88.265) (width 0.8) (layer "F.Cu") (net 12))
 (segment (start 91.44 88.265) (end 93.091 86.614) (width 0.8) (layer "F.Cu") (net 12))
 (segment (start 89.946 75.692) (end 88.422 75.692) (width 0.8) (layer "F.Cu") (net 12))
 (segment (start 93.741 79.487) (end 89.946 75.692) (width 0.8) (layer "F.Cu") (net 12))
 (segment (start 93.091 86.614) (end 96.206786 86.614) (width 0.8) (layer "F.Cu") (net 12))
 (segment (start 98.442 79.197214) (end 98.442001 84.378785) (width 0.8) (layer "F.Cu") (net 12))
 (segment (start 88.180472 93.228) (end 88.489 93.228) (width 0.8) (layer "F.Cu") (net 12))
 (segment (start 98.442001 84.378785) (end 96.206786 86.614) (width 0.8) (layer "F.Cu") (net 12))
 (segment (start 93.741 79.487) (end 93.741 79.038214) (width 0.8) (layer "F.Cu") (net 12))
 (segment (start 96.042 81.788) (end 93.741 79.487) (width 0.8) (layer "F.Cu") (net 12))
 (segment (start 86.689 89.639472) (end 88.063472 88.265) (width 0.8) (layer "F.Cu") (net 12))
 (segment (start 95.439214 77.34) (end 96.584786 77.34) (width 0.8) (layer "F.Cu") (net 12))
 (segment (start 96.584786 77.34) (end 98.442 79.197214) (width 0.8) (layer "F.Cu") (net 12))
 (segment (start 86.689 91.736528) (end 88.180472 93.228) (width 0.8) (layer "F.Cu") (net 12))
 (segment (start 93.741 79.038214) (end 95.439214 77.34) (width 0.8) (layer "F.Cu") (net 12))
 (segment (start 86.689 89.639472) (end 86.689 91.736528) (width 0.8) (layer "F.Cu") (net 12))
 (segment (start 92.192 90.688) (end 91.821 90.688) (width 0.8) (layer "F.Cu") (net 15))
 (segment (start 94.361 88.519) (end 92.192 90.688) (width 0.8) (layer "F.Cu") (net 15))
 (segment (start 91.821 90.688) (end 88.489 90.688) (width 0.8) (layer "F.Cu") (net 15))
 (segment (start 99.442001 78.292001) (end 99.442002 84.792998) (width 0.8) (layer "F.Cu") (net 15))
 (segment (start 98.044 93.345) (end 100.584 90.805) (width 0.8) (layer "F.Cu") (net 15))
 (segment (start 95.374 102.873) (end 98.044 100.203) (width 0.8) (layer "F.Cu") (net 15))
 (segment (start 96.842 75.692) (end 99.442001 78.292001) (width 0.8) (layer "F.Cu") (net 15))
 (segment (start 91.821 100.604786) (end 94.089214 102.873) (width 0.8) (layer "F.Cu") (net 15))
 (segment (start 99.442002 84.792998) (end 95.716 88.519) (width 0.8) (layer "F.Cu") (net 15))
 (segment (start 96.042 75.692) (end 96.842 75.692) (width 0.8) (layer "F.Cu") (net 15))
 (segment (start 98.044 100.203) (end 98.044 93.345) (width 0.8) (layer "F.Cu") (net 15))
 (segment (start 94.089214 102.873) (end 95.374 102.873) (width 0.8) (layer "F.Cu") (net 15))
 (segment (start 91.821 90.688) (end 91.821 100.604786) (width 0.8) (layer "F.Cu") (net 15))
 (segment (start 95.716 88.519) (end 94.361 88.519) (width 0.8) (layer "F.Cu") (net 15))
 (segment (start 137.678 94.029786) (end 134.552786 97.155) (width 0.8) (layer "F.Cu") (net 19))
 (segment (start 128.334688 93.977) (end 131.512688 97.155) (width 0.8) (layer "F.Cu") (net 19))
 (segment (start 99.134 99.007) (end 99.695 99.568) (width 0.8) (layer "F.Cu") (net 19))
 (segment (start 137.678 93.99) (end 137.678 94.029786) (width 0.8) (layer "F.Cu") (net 19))
 (segment (start 122.806 102.492) (end 125.222 100.076) (width 0.8) (layer "F.Cu") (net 19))
 (segment (start 134.552786 97.155) (end 131.512688 97.155) (width 0.8) (layer "F.Cu") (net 19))
 (segment (start 121.394214 102.492) (end 122.806 102.492) (width 0.8) (layer "F.Cu") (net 19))
 (segment (start 100.584 93.345) (end 102.105 91.824) (width 0.8) (layer "F.Cu") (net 19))
 (segment (start 115.737786 85.23) (end 120.177 89.669214) (width 0.8) (layer "F.Cu") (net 19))
 (segment (start 110.138 85.23) (end 115.737786 85.23) (width 0.8) (layer "F.Cu") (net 19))
 (segment (start 105.510786 92.078) (end 108.725 88.863786) (width 0.8) (layer "F.Cu") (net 19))
 (segment (start 120.177 89.669214) (end 120.177 101.274786) (width 0.8) (layer "F.Cu") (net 19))
 (segment (start 102.105 89.03) (end 103.505 87.63) (width 0.8) (layer "F.Cu") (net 19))
 (segment (start 100.584 93.345) (end 99.134 94.795) (width 0.8) (layer "F.Cu") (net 19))
 (segment (start 99.695 99.568) (end 100.584 99.568) (width 0.8) (layer "F.Cu") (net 19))
 (segment (start 125.222 94.920214) (end 125.222 100.076) (width 0.8) (layer "F.Cu") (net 19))
 (segment (start 126.165214 93.977) (end 125.222 94.920214) (width 0.8) (layer "F.Cu") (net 19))
 (segment (start 126.165214 93.977) (end 128.334688 93.977) (width 0.8) (layer "F.Cu") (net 19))
 (segment (start 100.584 93.345) (end 101.851 92.078) (width 0.8) (layer "F.Cu") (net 19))
 (segment (start 120.177 101.274786) (end 121.394214 102.492) (width 0.8) (layer "F.Cu") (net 19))
 (segment (start 101.851 92.078) (end 105.510786 92.078) (width 0.8) (layer "F.Cu") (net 19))
 (segment (start 108.725 88.863786) (end 108.724999 86.643001) (width 0.8) (layer "F.Cu") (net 19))
 (segment (start 108.724999 86.643001) (end 110.138 85.23) (width 0.8) (layer "F.Cu") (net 19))
 (segment (start 99.134 94.795) (end 99.134 99.007) (width 0.8) (layer "F.Cu") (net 19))
 (segment (start 102.105 91.824) (end 102.105 89.03) (width 0.8) (layer "F.Cu") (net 19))
 (segment (start 115.627 95.387) (end 112.811 92.571) (width 0.8) (layer "F.Cu") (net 7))
 (segment (start 112.811 89.316) (end 111.125 87.63) (width 0.8) (layer "F.Cu") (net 7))
 (segment (start 112.811 92.571) (end 112.811 89.316) (width 0.8) (layer "F.Cu") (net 7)))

